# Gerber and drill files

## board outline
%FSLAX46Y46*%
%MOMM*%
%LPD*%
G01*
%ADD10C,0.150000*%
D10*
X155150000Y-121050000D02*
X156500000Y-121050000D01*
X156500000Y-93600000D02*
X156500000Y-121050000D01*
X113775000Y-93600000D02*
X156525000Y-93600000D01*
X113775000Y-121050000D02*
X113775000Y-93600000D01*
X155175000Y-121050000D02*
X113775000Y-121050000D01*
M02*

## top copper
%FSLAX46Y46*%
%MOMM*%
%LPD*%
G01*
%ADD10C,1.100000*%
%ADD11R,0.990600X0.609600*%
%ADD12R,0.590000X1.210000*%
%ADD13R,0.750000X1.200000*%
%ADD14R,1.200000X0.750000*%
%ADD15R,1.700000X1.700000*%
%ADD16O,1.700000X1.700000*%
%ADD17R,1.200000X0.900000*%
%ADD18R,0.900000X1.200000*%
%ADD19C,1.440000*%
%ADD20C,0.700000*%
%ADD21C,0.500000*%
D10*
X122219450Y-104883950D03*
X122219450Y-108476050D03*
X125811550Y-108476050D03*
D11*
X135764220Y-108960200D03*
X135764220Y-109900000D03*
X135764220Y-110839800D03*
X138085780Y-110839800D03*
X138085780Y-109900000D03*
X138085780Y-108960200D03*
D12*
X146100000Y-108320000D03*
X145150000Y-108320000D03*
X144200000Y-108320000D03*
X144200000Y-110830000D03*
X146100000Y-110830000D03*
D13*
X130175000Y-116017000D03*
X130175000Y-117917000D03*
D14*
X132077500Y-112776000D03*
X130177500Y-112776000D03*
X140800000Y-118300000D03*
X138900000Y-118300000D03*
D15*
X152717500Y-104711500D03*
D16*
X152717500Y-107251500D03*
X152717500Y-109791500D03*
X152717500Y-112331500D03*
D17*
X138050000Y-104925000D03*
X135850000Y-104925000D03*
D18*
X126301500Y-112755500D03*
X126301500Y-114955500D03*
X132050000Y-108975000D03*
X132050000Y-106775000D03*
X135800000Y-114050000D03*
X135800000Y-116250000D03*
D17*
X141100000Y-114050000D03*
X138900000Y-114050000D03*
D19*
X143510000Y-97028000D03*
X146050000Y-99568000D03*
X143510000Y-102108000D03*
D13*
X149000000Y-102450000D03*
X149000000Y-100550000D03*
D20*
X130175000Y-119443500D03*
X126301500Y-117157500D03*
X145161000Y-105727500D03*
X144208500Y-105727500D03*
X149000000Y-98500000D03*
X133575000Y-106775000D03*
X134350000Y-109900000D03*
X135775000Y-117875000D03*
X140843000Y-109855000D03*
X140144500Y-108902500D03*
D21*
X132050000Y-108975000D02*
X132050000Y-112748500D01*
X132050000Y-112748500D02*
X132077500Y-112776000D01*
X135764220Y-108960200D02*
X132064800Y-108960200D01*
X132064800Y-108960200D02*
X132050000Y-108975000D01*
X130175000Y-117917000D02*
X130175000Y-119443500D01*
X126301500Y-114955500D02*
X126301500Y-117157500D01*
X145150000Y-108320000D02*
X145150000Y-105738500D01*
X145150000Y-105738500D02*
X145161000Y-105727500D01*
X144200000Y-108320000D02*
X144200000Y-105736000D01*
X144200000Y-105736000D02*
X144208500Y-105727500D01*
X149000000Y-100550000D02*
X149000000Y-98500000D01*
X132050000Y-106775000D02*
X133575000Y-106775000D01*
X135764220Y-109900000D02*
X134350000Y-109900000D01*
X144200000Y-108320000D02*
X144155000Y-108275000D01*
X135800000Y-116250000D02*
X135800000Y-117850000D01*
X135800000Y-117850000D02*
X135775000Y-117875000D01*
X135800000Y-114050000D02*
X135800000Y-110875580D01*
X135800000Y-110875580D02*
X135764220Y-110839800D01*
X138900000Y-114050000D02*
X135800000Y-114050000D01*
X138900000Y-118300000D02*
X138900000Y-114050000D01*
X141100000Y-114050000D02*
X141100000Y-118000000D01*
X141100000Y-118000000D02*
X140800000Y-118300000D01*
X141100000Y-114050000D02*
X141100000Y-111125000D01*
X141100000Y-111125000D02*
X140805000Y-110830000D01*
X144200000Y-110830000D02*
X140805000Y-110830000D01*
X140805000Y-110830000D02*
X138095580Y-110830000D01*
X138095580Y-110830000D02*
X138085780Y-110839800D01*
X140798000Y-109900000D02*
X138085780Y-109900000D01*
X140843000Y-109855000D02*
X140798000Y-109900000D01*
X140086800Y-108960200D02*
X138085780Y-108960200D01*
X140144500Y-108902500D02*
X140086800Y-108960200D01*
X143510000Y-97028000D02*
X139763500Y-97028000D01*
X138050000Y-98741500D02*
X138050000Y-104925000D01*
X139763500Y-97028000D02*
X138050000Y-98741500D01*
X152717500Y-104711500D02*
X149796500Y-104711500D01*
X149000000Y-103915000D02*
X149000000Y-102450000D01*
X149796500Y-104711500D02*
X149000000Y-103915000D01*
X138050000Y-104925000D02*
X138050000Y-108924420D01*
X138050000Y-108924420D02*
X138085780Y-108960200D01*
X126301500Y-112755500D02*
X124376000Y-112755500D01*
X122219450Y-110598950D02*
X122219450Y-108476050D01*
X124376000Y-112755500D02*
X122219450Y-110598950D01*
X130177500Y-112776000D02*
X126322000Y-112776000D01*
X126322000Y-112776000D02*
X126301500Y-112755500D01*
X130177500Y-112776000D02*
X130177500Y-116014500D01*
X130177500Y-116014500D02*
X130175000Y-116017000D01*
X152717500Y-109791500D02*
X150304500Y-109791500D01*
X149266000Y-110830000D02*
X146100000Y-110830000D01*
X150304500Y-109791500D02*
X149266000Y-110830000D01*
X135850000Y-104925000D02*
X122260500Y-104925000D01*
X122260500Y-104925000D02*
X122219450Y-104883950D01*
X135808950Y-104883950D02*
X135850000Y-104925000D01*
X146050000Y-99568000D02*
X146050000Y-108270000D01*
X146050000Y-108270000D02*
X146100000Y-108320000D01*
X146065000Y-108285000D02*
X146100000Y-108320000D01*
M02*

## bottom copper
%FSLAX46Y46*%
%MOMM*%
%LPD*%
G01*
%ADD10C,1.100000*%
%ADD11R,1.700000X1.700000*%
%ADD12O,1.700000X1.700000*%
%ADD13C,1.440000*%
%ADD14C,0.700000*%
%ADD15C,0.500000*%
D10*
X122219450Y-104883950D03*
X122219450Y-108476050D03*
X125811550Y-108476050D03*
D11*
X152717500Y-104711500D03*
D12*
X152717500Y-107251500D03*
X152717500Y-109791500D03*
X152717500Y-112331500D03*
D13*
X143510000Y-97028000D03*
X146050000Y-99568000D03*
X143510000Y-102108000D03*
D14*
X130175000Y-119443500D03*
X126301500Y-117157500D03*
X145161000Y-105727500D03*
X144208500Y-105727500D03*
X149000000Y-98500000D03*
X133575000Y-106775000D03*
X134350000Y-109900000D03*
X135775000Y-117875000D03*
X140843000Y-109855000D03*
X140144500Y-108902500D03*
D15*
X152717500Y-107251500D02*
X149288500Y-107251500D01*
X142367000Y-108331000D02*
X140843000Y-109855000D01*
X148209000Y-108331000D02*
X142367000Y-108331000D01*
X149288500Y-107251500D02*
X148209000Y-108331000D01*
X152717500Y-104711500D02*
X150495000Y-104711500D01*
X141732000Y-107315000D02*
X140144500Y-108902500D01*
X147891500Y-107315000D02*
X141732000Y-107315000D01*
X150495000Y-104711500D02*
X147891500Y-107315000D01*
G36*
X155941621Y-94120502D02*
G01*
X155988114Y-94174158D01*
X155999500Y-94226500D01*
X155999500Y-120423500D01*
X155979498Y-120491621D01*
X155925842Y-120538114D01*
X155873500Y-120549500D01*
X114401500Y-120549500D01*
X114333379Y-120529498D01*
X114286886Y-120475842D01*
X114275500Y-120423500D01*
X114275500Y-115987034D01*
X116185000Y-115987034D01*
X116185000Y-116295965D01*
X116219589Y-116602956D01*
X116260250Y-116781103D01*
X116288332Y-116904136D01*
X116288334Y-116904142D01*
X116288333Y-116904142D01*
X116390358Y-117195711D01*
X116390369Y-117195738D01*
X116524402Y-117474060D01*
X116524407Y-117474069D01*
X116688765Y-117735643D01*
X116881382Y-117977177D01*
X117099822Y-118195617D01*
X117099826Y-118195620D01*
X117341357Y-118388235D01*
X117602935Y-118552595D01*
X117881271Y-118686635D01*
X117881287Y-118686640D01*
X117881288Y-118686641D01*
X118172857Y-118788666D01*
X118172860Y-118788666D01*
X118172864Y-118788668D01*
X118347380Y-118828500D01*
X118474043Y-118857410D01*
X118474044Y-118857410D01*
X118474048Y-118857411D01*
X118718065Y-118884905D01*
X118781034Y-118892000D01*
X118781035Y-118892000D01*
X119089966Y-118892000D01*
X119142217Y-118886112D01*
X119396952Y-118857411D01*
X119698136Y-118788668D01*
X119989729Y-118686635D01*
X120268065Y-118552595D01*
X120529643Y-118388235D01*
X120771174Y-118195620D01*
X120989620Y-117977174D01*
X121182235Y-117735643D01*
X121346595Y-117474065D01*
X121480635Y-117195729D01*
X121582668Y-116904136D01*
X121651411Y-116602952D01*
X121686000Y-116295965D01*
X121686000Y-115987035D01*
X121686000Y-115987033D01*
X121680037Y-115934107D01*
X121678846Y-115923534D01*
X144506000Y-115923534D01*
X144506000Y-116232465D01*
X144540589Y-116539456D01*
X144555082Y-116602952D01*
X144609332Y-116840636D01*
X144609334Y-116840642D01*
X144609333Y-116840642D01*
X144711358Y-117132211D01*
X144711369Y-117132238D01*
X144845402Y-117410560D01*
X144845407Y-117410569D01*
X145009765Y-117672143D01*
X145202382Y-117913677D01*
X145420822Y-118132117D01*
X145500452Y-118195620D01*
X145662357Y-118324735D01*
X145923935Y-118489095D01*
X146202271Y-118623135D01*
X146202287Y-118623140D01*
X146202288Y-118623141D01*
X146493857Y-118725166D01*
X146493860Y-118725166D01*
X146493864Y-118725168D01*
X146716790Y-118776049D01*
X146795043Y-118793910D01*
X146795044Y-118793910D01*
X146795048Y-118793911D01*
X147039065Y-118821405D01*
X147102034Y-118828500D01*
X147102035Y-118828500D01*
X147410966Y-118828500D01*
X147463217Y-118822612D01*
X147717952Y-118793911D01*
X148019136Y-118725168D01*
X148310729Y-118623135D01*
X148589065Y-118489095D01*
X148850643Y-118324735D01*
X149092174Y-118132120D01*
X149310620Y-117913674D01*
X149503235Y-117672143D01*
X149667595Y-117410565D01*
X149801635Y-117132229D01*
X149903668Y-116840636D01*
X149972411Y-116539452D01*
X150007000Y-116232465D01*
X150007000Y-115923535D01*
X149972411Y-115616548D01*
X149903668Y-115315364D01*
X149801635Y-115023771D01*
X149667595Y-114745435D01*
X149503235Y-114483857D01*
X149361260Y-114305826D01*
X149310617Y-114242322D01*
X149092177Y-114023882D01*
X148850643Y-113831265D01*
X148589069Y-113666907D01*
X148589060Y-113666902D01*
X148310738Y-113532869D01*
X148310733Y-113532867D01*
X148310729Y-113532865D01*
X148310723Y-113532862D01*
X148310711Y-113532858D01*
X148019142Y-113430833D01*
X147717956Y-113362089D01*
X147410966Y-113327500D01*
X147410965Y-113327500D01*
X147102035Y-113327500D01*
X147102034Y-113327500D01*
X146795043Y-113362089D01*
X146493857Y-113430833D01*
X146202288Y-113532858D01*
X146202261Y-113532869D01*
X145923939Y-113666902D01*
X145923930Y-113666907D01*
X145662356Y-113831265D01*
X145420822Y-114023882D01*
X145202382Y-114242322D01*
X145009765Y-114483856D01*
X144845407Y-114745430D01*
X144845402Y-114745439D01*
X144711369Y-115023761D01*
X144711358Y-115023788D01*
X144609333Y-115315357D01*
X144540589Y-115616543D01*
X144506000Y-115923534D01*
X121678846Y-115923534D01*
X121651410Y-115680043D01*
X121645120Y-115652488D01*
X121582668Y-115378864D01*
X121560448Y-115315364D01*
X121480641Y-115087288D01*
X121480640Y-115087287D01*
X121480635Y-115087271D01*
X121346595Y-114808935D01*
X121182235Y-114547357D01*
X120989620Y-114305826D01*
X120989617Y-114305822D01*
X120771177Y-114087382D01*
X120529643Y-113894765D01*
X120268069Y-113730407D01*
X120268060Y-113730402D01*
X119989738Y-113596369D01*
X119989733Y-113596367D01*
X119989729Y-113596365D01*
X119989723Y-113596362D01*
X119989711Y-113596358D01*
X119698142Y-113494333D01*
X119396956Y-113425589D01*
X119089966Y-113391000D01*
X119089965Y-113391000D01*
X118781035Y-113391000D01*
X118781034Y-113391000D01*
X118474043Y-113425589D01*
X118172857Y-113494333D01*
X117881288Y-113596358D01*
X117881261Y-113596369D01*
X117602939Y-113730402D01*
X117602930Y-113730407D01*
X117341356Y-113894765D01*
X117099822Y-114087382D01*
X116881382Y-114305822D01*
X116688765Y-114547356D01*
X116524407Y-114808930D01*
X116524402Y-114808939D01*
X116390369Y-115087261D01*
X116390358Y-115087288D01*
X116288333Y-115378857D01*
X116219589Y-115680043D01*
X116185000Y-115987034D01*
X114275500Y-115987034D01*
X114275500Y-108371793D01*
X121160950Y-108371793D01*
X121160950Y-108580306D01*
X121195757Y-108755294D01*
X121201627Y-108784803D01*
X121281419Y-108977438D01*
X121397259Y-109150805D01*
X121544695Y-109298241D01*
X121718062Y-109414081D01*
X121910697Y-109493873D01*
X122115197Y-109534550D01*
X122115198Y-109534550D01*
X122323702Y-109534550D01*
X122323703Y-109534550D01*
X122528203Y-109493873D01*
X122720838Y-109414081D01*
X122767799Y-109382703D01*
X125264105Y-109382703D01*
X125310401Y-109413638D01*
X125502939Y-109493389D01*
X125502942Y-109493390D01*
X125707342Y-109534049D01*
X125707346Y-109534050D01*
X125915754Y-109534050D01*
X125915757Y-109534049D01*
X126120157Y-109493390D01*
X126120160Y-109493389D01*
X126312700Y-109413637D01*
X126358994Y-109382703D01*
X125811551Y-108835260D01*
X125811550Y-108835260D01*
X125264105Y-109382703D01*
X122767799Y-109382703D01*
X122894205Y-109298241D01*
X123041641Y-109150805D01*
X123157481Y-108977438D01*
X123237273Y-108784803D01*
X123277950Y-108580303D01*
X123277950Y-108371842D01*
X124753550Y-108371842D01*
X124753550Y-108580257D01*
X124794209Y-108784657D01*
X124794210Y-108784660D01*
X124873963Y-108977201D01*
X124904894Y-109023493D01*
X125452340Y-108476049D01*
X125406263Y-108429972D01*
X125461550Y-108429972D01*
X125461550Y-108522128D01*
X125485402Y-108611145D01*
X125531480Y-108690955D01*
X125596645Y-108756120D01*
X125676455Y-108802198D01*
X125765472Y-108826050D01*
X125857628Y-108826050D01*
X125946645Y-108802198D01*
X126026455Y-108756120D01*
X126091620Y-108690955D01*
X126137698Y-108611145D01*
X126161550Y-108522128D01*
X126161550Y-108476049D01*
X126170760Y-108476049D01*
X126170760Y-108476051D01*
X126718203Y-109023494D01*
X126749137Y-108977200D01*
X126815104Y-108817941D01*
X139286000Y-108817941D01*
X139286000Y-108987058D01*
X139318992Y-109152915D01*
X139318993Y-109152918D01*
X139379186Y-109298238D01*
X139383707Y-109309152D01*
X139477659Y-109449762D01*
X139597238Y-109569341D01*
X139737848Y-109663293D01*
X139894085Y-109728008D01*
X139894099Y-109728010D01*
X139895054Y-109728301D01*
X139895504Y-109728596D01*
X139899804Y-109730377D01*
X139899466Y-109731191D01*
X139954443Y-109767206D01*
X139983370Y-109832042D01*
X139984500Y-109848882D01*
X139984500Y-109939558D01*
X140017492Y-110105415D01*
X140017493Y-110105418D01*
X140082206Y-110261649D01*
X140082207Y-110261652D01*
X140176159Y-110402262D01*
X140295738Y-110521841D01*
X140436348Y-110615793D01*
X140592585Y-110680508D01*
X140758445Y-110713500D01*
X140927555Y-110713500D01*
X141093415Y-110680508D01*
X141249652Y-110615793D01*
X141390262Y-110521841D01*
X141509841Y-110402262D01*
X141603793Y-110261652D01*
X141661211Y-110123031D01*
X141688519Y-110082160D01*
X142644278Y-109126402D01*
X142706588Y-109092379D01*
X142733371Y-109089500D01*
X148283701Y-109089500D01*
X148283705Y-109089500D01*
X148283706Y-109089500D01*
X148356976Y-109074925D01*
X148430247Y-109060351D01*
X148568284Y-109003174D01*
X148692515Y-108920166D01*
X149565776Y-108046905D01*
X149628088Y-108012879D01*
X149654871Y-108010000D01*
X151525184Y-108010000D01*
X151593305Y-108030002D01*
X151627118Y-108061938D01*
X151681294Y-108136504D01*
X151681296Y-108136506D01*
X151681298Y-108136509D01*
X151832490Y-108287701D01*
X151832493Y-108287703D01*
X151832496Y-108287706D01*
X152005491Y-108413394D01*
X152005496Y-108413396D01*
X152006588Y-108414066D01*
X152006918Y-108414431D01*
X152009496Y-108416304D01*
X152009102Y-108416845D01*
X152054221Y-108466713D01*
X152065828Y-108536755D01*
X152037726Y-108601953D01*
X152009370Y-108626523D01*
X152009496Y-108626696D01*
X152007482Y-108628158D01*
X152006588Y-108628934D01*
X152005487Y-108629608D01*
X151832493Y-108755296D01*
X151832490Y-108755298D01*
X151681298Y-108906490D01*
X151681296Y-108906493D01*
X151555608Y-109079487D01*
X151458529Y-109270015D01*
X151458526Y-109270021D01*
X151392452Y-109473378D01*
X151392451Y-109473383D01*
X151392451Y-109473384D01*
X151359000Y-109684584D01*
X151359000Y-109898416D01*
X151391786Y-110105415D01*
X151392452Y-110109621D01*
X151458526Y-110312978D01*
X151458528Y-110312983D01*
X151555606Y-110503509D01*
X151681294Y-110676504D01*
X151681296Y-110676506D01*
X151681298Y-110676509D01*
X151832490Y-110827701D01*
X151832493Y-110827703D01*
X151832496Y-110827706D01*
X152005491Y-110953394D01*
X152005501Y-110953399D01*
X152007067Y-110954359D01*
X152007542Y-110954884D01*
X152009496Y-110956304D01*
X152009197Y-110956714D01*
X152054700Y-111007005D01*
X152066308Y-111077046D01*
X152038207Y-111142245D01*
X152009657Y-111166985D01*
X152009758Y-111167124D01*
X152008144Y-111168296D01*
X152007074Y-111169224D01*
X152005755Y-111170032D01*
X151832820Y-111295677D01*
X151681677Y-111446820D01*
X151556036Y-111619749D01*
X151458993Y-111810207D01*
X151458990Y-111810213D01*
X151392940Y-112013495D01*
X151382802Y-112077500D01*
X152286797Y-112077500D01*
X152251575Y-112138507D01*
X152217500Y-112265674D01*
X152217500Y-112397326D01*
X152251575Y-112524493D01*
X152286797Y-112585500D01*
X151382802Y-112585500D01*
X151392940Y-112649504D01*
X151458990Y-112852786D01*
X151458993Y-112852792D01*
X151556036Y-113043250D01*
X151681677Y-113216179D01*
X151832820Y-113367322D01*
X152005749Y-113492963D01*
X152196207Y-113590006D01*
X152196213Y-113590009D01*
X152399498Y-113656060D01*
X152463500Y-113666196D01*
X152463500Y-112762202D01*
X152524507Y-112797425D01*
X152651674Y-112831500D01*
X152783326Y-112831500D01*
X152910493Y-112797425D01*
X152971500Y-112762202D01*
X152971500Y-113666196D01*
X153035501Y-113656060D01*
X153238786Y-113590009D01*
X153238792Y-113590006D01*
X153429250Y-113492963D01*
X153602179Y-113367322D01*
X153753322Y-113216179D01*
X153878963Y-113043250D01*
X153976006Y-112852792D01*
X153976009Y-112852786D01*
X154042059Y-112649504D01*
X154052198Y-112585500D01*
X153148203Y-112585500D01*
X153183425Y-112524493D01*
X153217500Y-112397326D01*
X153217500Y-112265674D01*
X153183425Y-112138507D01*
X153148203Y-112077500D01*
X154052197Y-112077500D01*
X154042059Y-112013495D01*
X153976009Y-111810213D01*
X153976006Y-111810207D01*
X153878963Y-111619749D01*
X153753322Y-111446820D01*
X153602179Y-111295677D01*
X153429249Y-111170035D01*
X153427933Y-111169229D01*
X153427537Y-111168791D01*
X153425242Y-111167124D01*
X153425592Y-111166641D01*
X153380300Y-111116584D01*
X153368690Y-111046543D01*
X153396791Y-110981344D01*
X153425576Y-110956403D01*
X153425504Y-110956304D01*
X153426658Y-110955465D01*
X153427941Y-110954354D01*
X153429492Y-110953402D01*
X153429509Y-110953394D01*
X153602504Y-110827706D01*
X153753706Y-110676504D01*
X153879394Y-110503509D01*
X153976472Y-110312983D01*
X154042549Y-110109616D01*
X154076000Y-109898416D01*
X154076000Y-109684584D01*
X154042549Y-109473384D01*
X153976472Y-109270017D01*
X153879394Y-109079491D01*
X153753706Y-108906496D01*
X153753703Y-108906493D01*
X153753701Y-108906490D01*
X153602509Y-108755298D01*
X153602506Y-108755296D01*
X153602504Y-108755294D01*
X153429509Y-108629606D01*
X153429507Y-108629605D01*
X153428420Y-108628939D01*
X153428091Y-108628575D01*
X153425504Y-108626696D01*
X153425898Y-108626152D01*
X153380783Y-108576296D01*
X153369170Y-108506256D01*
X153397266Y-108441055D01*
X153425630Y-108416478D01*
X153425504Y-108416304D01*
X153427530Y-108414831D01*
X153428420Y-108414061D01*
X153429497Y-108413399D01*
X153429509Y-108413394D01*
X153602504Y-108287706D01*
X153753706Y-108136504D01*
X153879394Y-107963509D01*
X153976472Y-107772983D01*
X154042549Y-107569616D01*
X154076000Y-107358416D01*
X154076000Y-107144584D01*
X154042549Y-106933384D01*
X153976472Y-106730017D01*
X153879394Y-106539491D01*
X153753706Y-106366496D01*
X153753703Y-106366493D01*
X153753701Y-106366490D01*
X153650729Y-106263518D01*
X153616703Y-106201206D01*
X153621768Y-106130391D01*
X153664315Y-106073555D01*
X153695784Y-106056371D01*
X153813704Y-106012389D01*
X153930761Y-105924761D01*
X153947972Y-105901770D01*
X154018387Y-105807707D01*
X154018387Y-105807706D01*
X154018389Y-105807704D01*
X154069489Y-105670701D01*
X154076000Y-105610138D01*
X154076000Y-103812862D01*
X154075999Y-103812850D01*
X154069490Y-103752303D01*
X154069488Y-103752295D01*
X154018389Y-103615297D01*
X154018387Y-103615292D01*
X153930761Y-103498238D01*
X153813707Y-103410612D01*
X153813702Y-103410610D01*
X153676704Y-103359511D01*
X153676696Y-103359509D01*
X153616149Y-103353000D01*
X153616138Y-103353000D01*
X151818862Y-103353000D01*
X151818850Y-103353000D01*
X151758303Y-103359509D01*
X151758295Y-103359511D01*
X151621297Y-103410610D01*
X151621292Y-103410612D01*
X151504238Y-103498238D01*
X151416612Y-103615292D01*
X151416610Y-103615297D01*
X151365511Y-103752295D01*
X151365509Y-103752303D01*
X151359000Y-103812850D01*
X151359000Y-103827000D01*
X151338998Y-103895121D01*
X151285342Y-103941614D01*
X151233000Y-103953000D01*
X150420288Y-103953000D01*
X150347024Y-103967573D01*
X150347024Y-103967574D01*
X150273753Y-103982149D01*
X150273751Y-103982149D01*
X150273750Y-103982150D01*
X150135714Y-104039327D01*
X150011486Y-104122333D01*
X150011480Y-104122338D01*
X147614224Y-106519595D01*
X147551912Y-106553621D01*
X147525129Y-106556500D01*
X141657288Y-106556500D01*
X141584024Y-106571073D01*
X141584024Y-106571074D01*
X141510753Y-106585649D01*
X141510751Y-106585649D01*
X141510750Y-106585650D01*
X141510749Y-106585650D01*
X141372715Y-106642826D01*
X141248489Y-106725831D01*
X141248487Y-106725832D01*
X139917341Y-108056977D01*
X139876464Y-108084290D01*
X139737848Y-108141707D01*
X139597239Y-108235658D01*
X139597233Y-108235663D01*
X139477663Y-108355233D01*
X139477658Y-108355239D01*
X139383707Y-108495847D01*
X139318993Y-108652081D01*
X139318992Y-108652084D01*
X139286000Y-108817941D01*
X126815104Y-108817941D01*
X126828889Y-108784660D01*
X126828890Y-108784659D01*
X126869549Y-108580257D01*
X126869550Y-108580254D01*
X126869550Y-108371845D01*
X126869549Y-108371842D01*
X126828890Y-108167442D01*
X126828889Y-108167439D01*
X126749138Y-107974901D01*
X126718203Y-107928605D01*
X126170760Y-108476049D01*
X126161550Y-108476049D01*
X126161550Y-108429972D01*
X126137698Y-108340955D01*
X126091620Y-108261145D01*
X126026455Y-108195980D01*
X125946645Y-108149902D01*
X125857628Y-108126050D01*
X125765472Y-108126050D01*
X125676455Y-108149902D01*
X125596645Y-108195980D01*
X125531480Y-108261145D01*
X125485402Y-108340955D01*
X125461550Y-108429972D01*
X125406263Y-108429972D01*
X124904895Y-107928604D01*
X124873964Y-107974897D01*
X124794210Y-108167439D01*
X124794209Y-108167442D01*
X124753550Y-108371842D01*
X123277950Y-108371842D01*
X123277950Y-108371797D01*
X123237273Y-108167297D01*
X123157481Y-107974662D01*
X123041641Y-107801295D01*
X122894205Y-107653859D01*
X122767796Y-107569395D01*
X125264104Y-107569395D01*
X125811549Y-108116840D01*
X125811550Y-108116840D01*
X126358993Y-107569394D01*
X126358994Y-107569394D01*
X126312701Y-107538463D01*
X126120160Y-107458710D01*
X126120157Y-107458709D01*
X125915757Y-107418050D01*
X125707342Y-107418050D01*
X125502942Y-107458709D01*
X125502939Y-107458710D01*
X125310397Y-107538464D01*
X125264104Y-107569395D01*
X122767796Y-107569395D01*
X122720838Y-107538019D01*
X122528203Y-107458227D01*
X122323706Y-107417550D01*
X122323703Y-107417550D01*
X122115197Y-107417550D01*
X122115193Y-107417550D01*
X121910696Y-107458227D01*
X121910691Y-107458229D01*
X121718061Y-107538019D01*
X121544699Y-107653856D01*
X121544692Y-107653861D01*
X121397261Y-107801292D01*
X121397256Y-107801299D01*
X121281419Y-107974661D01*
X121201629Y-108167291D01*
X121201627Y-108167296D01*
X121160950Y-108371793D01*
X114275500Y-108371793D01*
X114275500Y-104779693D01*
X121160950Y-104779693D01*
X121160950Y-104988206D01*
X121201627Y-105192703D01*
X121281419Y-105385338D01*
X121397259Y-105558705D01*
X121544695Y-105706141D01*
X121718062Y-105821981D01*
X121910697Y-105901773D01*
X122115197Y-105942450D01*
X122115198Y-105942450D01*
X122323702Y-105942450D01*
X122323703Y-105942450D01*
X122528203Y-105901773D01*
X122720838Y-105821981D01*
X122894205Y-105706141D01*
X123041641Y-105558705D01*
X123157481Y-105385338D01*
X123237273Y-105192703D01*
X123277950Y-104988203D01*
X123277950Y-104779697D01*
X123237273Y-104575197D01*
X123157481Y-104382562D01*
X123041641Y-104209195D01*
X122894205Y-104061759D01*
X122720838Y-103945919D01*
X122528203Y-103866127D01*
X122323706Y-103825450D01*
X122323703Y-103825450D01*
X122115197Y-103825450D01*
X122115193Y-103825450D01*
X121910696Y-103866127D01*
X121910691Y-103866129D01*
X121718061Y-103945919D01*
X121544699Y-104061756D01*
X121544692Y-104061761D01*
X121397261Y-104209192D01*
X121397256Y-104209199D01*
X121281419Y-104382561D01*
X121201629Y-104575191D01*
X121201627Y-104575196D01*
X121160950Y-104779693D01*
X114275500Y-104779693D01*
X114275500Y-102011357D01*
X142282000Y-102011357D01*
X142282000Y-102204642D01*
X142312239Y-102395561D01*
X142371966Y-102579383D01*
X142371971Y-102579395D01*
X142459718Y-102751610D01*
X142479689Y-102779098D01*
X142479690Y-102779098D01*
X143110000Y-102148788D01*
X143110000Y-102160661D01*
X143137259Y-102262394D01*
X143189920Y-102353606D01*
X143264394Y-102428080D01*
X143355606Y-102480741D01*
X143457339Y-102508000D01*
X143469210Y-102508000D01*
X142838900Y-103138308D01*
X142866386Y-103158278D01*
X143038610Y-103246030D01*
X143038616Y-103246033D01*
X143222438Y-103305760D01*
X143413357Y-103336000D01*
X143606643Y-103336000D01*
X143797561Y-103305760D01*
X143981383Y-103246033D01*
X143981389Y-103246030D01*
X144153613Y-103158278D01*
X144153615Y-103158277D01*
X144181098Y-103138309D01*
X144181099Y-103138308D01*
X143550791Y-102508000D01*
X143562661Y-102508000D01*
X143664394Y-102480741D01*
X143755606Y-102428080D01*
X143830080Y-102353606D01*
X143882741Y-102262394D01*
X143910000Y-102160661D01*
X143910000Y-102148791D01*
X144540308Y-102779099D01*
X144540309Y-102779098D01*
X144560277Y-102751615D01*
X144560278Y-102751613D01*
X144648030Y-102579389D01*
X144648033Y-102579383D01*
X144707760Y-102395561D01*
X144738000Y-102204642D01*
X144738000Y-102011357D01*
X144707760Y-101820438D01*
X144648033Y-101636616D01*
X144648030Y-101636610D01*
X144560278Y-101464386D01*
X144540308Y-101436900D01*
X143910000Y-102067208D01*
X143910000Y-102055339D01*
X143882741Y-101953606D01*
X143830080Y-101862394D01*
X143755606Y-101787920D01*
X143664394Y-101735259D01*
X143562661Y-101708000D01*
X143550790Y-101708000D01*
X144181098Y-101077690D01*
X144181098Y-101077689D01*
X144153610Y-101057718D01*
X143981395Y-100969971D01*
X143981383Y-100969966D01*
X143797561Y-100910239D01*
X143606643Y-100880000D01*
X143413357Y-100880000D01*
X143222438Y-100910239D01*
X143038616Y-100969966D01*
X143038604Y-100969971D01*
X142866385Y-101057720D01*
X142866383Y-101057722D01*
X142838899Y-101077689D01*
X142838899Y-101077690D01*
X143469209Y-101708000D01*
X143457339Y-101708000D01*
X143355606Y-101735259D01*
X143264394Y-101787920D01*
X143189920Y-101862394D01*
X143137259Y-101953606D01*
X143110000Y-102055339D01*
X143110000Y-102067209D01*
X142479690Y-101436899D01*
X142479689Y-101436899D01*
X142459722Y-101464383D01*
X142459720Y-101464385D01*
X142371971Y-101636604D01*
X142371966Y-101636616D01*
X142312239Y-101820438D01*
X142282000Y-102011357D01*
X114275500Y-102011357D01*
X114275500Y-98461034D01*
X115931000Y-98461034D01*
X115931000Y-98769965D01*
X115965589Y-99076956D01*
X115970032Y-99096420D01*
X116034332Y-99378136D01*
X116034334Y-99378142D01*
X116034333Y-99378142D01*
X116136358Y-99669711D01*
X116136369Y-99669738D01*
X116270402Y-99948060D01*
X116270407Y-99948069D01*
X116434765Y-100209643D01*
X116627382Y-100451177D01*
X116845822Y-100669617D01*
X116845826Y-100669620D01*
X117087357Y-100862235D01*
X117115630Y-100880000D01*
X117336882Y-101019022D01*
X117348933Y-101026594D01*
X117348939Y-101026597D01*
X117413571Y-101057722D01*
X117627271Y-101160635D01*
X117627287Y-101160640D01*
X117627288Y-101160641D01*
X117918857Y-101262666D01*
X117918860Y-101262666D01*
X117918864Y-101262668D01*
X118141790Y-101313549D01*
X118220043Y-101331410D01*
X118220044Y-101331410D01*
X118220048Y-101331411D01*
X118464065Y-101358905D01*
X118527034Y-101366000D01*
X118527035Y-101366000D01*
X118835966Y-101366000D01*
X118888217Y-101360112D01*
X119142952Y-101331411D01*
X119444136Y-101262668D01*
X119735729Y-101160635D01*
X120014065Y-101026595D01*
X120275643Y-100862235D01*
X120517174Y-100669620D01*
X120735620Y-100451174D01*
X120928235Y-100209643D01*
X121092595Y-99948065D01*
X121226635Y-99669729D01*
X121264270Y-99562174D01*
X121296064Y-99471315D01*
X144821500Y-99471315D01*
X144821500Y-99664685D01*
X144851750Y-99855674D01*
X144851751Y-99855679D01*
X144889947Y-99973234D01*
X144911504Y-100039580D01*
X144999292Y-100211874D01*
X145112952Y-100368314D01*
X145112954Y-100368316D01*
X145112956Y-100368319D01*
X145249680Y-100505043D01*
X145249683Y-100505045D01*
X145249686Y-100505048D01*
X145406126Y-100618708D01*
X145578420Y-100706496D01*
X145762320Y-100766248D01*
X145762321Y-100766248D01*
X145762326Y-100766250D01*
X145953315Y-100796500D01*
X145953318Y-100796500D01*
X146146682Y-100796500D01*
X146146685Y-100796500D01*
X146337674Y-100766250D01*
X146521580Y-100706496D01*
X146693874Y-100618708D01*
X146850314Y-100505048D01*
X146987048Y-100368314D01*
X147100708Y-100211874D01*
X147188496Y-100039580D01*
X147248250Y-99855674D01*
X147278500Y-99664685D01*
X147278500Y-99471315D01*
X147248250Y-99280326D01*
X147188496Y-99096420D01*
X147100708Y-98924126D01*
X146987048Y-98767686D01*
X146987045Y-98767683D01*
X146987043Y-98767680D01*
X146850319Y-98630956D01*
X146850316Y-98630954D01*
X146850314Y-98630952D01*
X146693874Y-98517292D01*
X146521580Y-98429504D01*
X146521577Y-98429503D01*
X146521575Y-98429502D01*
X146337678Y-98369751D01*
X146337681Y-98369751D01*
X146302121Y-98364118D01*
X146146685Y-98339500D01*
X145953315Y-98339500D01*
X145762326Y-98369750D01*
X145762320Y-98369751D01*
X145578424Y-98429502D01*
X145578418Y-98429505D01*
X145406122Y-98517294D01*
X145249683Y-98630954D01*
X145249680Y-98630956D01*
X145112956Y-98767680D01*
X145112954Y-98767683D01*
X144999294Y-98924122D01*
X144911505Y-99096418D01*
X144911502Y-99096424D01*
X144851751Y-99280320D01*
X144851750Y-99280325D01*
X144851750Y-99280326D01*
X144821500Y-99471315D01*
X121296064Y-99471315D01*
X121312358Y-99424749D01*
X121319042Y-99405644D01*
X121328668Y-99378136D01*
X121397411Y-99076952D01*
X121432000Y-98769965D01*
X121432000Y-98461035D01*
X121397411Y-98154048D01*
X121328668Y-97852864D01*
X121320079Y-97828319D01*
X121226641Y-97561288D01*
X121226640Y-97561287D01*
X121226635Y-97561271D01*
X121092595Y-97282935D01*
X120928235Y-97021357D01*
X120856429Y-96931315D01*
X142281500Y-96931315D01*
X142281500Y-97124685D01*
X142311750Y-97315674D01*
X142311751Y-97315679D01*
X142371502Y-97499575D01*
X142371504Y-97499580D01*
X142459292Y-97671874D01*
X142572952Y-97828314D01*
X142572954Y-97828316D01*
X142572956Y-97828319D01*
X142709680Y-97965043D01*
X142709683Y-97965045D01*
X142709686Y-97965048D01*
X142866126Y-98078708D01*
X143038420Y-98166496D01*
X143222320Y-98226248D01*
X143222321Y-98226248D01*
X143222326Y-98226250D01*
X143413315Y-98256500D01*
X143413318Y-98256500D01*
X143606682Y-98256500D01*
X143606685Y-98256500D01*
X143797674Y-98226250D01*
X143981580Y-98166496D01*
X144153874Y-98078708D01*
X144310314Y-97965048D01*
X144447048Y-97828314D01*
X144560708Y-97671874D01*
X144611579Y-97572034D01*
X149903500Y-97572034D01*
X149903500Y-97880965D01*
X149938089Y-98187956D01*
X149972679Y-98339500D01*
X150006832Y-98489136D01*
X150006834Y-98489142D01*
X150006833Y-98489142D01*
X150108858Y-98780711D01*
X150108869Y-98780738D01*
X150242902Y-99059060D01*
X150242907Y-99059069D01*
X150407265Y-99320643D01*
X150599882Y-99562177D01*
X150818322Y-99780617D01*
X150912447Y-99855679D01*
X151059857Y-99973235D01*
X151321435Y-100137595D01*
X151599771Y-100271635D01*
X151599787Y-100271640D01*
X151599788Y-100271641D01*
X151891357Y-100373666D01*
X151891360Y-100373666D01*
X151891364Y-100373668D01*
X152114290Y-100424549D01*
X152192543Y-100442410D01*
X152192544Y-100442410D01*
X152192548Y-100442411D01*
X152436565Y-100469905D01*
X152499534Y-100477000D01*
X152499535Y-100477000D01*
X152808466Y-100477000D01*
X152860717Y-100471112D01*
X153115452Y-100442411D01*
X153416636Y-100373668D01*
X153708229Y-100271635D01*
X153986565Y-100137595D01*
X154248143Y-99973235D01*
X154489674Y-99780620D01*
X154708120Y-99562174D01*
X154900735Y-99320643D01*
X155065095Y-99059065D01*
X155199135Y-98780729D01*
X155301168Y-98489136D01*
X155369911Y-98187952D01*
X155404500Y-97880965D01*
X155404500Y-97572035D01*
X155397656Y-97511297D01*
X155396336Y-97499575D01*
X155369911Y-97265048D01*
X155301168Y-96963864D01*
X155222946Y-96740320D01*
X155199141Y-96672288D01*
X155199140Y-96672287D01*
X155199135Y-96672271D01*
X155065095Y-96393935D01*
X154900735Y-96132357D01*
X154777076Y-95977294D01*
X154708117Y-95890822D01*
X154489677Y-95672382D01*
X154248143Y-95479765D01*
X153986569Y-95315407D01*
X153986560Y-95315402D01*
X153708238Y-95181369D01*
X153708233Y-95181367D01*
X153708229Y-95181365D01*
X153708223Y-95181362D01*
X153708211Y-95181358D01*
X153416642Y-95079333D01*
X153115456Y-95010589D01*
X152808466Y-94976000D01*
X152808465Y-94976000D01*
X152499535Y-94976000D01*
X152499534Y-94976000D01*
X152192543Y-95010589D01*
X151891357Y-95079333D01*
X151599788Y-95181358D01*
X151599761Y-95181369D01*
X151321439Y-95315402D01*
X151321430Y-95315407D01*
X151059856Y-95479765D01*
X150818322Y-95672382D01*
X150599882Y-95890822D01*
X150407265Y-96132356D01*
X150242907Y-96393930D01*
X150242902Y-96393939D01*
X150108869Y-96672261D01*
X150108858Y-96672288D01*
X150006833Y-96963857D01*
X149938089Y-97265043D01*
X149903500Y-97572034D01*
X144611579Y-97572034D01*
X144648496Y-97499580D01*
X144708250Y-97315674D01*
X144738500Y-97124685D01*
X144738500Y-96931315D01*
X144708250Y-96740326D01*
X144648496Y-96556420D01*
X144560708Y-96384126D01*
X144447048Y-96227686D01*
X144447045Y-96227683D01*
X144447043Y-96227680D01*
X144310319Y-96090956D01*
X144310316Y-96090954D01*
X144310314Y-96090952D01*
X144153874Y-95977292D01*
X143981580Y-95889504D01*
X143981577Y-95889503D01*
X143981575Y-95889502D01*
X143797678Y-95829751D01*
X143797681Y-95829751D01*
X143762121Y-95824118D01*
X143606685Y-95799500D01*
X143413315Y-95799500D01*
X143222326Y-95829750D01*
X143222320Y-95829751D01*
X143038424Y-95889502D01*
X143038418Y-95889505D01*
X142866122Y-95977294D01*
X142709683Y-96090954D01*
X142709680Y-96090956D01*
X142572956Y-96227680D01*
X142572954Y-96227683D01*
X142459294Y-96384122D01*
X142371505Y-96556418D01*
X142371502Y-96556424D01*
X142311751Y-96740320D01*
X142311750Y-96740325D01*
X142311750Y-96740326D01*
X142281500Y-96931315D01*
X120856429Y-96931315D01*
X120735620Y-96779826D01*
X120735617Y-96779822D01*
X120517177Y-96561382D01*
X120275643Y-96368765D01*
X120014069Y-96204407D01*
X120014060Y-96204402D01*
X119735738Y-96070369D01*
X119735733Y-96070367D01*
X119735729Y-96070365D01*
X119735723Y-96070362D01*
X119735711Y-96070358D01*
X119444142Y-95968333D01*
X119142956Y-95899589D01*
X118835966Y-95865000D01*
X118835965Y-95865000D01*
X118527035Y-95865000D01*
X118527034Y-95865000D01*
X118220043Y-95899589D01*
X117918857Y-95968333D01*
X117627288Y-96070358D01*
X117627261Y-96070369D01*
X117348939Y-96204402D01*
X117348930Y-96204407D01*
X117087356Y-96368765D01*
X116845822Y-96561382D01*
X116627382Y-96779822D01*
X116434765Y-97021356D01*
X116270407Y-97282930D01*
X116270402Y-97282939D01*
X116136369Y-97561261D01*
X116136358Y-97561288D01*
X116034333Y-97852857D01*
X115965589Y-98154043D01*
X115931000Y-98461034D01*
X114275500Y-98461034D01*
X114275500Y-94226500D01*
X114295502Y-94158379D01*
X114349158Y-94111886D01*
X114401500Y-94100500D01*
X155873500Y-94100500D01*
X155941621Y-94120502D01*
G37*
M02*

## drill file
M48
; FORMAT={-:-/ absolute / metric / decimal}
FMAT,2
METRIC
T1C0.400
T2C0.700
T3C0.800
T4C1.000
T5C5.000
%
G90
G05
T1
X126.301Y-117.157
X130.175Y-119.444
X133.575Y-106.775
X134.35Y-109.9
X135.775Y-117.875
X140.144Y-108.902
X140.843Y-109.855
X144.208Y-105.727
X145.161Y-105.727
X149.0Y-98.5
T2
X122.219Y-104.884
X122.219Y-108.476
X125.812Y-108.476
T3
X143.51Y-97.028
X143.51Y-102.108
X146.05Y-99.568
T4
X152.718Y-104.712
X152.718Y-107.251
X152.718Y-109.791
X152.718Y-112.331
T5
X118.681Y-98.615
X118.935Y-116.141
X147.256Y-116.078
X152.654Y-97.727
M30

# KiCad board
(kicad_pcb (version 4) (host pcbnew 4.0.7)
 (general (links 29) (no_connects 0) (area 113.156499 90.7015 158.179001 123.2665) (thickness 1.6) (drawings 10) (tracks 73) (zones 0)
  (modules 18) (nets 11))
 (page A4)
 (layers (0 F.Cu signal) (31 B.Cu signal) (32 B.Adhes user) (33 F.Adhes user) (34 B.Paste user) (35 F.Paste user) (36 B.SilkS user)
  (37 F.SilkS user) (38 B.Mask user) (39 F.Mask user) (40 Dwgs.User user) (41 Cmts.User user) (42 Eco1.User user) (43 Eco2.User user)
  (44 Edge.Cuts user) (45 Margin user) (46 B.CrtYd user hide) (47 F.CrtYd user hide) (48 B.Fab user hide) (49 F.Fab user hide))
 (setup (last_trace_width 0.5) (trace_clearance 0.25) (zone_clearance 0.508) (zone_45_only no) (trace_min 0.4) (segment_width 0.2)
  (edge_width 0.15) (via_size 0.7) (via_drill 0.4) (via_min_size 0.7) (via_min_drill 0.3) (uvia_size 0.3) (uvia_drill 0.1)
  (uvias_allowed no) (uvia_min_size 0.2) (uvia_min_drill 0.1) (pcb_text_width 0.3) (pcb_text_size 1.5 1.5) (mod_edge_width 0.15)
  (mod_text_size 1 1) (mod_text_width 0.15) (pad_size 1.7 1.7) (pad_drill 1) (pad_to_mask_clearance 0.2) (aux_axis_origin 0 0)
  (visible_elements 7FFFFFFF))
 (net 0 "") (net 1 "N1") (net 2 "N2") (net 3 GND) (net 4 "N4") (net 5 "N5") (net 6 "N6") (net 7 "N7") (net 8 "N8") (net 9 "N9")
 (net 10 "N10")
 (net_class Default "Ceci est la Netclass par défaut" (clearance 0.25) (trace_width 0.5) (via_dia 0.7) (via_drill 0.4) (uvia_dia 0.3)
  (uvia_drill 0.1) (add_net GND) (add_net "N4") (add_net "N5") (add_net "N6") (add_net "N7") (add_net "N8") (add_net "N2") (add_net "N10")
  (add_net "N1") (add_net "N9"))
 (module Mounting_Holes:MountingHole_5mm (layer F.Cu) (at 147.2565 116.078)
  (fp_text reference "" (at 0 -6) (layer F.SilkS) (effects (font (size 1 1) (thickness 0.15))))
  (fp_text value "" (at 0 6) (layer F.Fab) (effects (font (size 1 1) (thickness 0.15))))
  (pad 1 np_thru_hole circle (at 0 0) (size 5 5) (drill 5) (layers *.Cu *.Mask)))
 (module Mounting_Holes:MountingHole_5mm (layer F.Cu) (at 152.654 97.7265)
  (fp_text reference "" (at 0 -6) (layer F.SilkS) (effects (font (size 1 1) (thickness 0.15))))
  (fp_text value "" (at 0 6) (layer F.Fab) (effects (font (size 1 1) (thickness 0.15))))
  (pad 1 np_thru_hole circle (at 0 0) (size 5 5) (drill 5) (layers *.Cu *.Mask)))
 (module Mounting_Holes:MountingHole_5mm (layer F.Cu) (at 118.9355 116.1415)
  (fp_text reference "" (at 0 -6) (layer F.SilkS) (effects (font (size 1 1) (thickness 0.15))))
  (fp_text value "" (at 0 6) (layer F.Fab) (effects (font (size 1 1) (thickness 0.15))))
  (pad 1 np_thru_hole circle (at 0 0) (size 5 5) (drill 5) (layers *.Cu *.Mask)))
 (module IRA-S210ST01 (layer F.Cu) (at 124.0155 106.68 270)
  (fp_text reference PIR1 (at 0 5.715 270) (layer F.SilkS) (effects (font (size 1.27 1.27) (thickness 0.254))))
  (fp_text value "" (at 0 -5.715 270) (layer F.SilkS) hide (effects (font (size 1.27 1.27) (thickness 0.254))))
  (pad 1 thru_hole circle (at -1.79605 1.79605) (size 1.1 1.1) (drill 0.7) (layers *.Cu *.Mask F.SilkS) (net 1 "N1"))
  (pad 2 thru_hole circle (at 1.79605 1.79605) (size 1.1 1.1) (drill 0.7) (layers *.Cu *.Mask F.SilkS) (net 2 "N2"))
  (pad 3 thru_hole circle (at 1.79605 -1.79605) (size 1.1 1.1) (drill 0.7) (layers *.Cu *.Mask F.SilkS) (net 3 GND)))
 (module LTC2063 (layer F.Cu) (at 136.925 109.9)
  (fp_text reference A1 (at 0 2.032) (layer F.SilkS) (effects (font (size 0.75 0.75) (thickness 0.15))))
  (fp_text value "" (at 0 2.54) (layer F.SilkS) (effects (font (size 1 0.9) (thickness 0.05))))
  (pad 1 smd rect (at -1.16078 -0.9398) (size 0.9906 0.6096) (layers F.Cu F.Paste F.Mask) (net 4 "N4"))
  (pad 2 smd rect (at -1.16078 0) (size 0.9906 0.6096) (layers F.Cu F.Paste F.Mask) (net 3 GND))
  (pad 3 smd rect (at -1.16078 0.9398) (size 0.9906 0.6096) (layers F.Cu F.Paste F.Mask) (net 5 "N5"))
  (pad 4 smd rect (at 1.16078 0.9398) (size 0.9906 0.6096) (layers F.Cu F.Paste F.Mask) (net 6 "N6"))
  (pad 5 smd rect (at 1.16078 0) (size 0.9906 0.6096) (layers F.Cu F.Paste F.Mask) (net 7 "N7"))
  (pad 6 smd rect (at 1.16078 -0.9398) (size 0.9906 0.6096) (layers F.Cu F.Paste F.Mask) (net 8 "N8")))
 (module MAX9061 (layer F.Cu) (at 145.15 109.575 270)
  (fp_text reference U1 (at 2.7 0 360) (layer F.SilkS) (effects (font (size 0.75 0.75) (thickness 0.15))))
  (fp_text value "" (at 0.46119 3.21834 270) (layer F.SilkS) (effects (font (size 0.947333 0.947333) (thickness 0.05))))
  (pad 1 smd rect (at -1.255 -0.95 90) (size 1.21 0.59) (layers F.Cu F.Paste F.Mask) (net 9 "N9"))
  (pad 2 smd rect (at -1.255 0 90) (size 1.21 0.59) (layers F.Cu F.Paste F.Mask) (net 3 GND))
  (pad 3 smd rect (at -1.255 0.95 90) (size 1.21 0.59) (layers F.Cu F.Paste F.Mask) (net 3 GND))
  (pad 4 smd rect (at 1.255 0.95 270) (size 1.21 0.59) (layers F.Cu F.Paste F.Mask) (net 6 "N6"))
  (pad 5 smd rect (at 1.255 -0.95 270) (size 1.21 0.59) (layers F.Cu F.Paste F.Mask) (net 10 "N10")))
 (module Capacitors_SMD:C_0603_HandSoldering (layer F.Cu) (at 130.175 116.967 270)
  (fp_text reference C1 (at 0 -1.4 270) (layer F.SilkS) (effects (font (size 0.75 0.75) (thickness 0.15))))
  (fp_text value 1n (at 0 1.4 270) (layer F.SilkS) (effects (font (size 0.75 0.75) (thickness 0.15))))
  (pad 1 smd rect (at -0.95 0 270) (size 1.2 0.75) (layers F.Cu F.Paste F.Mask) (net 2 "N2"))
  (pad 2 smd rect (at 0.95 0 270) (size 1.2 0.75) (layers F.Cu F.Paste F.Mask) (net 3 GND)))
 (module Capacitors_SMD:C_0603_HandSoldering (layer F.Cu) (at 131.1275 112.776 180)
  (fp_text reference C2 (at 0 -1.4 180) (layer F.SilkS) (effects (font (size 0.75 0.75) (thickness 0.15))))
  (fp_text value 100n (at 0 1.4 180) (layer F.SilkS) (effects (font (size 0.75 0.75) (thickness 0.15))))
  (pad 1 smd rect (at -0.95 0 180) (size 1.2 0.75) (layers F.Cu F.Paste F.Mask) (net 4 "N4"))
  (pad 2 smd rect (at 0.95 0 180) (size 1.2 0.75) (layers F.Cu F.Paste F.Mask) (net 2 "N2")))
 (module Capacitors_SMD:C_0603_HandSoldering (layer F.Cu) (at 139.85 118.3 180)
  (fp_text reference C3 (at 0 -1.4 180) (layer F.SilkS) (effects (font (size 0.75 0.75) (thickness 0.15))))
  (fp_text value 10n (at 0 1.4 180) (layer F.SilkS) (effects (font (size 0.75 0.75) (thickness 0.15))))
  (pad 1 smd rect (at -0.95 0 180) (size 1.2 0.75) (layers F.Cu F.Paste F.Mask) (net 6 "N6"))
  (pad 2 smd rect (at 0.95 0 180) (size 1.2 0.75) (layers F.Cu F.Paste F.Mask) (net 5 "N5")))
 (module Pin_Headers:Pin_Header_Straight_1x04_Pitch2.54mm (layer F.Cu) (at 152.7175 104.7115)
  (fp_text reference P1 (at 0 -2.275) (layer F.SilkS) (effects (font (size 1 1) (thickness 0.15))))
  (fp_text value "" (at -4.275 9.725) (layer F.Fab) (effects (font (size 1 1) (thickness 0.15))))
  (pad 1 thru_hole rect (at 0 0) (size 1.7 1.7) (drill 1) (layers *.Cu *.Mask) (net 8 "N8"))
  (pad 2 thru_hole oval (at 0 2.54) (size 1.7 1.7) (drill 1) (layers *.Cu *.Mask) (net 7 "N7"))
  (pad 3 thru_hole oval (at 0 5.08) (size 1.7 1.7) (drill 1) (layers *.Cu *.Mask) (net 10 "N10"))
  (pad 4 thru_hole oval (at 0 7.62) (size 1.7 1.7) (drill 1) (layers *.Cu *.Mask) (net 3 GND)))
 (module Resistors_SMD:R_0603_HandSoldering (layer F.Cu) (at 136.95 104.925 180)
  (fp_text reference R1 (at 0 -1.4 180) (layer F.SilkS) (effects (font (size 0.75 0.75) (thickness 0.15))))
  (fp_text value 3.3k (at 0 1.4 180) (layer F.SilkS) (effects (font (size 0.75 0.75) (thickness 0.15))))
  (pad 1 smd rect (at -1.1 0 180) (size 1.2 0.9) (layers F.Cu F.Paste F.Mask) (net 8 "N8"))
  (pad 2 smd rect (at 1.1 0 180) (size 1.2 0.9) (layers F.Cu F.Paste F.Mask) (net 1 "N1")))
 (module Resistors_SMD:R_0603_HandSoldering (layer F.Cu) (at 126.3015 113.8555 270)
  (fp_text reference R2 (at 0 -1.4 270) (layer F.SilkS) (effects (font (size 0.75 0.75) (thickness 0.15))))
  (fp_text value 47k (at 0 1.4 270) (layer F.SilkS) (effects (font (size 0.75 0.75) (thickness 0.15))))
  (pad 1 smd rect (at -1.1 0 270) (size 1.2 0.9) (layers F.Cu F.Paste F.Mask) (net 2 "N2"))
  (pad 2 smd rect (at 1.1 0 270) (size 1.2 0.9) (layers F.Cu F.Paste F.Mask) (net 3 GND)))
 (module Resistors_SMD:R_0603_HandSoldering (layer F.Cu) (at 132.05 107.875 90)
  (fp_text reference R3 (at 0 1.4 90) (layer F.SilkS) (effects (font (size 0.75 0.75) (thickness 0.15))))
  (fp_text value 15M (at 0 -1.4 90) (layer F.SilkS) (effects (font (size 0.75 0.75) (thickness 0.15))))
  (pad 1 smd rect (at -1.1 0 90) (size 1.2 0.9) (layers F.Cu F.Paste F.Mask) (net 4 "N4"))
  (pad 2 smd rect (at 1.1 0 90) (size 1.2 0.9) (layers F.Cu F.Paste F.Mask) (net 3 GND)))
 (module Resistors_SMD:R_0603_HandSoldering (layer F.Cu) (at 135.8 115.15 270)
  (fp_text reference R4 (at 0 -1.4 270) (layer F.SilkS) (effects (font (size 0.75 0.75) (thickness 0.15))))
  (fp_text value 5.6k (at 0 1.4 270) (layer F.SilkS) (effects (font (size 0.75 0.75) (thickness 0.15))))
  (pad 1 smd rect (at -1.1 0 270) (size 1.2 0.9) (layers F.Cu F.Paste F.Mask) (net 5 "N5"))
  (pad 2 smd rect (at 1.1 0 270) (size 1.2 0.9) (layers F.Cu F.Paste F.Mask) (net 3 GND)))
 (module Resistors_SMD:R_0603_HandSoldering (layer F.Cu) (at 140 114.05 180)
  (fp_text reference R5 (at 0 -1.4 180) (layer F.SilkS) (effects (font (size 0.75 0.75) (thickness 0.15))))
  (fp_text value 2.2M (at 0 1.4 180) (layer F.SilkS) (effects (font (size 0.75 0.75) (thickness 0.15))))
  (pad 1 smd rect (at -1.1 0 180) (size 1.2 0.9) (layers F.Cu F.Paste F.Mask) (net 6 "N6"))
  (pad 2 smd rect (at 1.1 0 180) (size 1.2 0.9) (layers F.Cu F.Paste F.Mask) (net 5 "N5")))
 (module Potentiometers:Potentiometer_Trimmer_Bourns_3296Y (layer F.Cu) (at 143.51 97.028 90)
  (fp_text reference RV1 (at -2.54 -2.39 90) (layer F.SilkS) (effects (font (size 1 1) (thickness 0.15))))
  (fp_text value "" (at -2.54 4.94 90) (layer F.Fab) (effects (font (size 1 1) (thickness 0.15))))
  (pad 1 thru_hole circle (at 0 0 90) (size 1.44 1.44) (drill 0.8) (layers *.Cu *.Mask) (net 8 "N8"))
  (pad 2 thru_hole circle (at -2.54 2.54 90) (size 1.44 1.44) (drill 0.8) (layers *.Cu *.Mask) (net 9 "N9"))
  (pad 3 thru_hole circle (at -5.08 0 90) (size 1.44 1.44) (drill 0.8) (layers *.Cu *.Mask) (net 3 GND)))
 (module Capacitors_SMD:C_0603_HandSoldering (layer F.Cu) (at 149 101.5 90)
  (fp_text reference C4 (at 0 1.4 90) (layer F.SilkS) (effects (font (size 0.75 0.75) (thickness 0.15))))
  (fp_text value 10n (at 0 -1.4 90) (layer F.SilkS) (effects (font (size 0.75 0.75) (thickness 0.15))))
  (pad 1 smd rect (at -0.95 0 90) (size 1.2 0.75) (layers F.Cu F.Paste F.Mask) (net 8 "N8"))
  (pad 2 smd rect (at 0.95 0 90) (size 1.2 0.75) (layers F.Cu F.Paste F.Mask) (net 3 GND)))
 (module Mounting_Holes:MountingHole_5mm (layer F.Cu) (at 118.6815 98.6155)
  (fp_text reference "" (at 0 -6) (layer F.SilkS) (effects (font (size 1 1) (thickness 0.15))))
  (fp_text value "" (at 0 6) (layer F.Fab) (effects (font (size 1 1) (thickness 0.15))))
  (pad 1 np_thru_hole circle (at 0 0) (size 5 5) (drill 5) (layers *.Cu *.Mask)))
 (gr_line (start 155.15 121.05) (end 156.5 121.05) (angle 90) (layer Edge.Cuts) (width 0.15))
 (gr_line (start 156.5 93.6) (end 156.5 121.05) (angle 90) (layer Edge.Cuts) (width 0.15))
 (gr_line (start 113.775 93.6) (end 156.525 93.6) (angle 90) (layer Edge.Cuts) (width 0.15))
 (gr_line (start 113.775 121.05) (end 113.775 93.6) (angle 90) (layer Edge.Cuts) (width 0.15))
 (gr_line (start 155.175 121.05) (end 113.775 121.05) (angle 90) (layer Edge.Cuts) (width 0.15))
 (segment (start 132.05 108.975) (end 132.05 112.7485) (width 0.5) (layer F.Cu) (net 4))
 (segment (start 132.05 112.7485) (end 132.0775 112.776) (width 0.5) (layer F.Cu) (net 4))
 (segment (start 135.76422 108.9602) (end 132.0648 108.9602) (width 0.5) (layer F.Cu) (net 4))
 (segment (start 132.0648 108.9602) (end 132.05 108.975) (width 0.5) (layer F.Cu) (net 4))
 (segment (start 130.175 117.917) (end 130.175 119.4435) (width 0.5) (layer F.Cu) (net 3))
 (via (at 130.175 119.4435) (size 0.7) (drill 0.4) (layers F.Cu B.Cu) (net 3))
 (segment (start 126.3015 114.9555) (end 126.3015 117.1575) (width 0.5) (layer F.Cu) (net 3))
 (via (at 126.3015 117.1575) (size 0.7) (drill 0.4) (layers F.Cu B.Cu) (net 3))
 (segment (start 145.15 108.32) (end 145.15 105.7385) (width 0.5) (layer F.Cu) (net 3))
 (via (at 145.161 105.7275) (size 0.7) (drill 0.4) (layers F.Cu B.Cu) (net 3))
 (segment (start 145.15 105.7385) (end 145.161 105.7275) (width 0.5) (layer F.Cu) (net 3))
 (segment (start 144.2 108.32) (end 144.2 105.736) (width 0.5) (layer F.Cu) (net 3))
 (via (at 144.2085 105.7275) (size 0.7) (drill 0.4) (layers F.Cu B.Cu) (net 3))
 (segment (start 144.2 105.736) (end 144.2085 105.7275) (width 0.5) (layer F.Cu) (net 3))
 (segment (start 149 100.55) (end 149 98.5) (width 0.5) (layer F.Cu) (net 3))
 (via (at 149 98.5) (size 0.7) (drill 0.4) (layers F.Cu B.Cu) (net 3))
 (segment (start 132.05 106.775) (end 133.575 106.775) (width 0.5) (layer F.Cu) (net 3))
 (via (at 133.575 106.775) (size 0.7) (drill 0.4) (layers F.Cu B.Cu) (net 3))
 (segment (start 135.76422 109.9) (end 134.35 109.9) (width 0.5) (layer F.Cu) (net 3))
 (via (at 134.35 109.9) (size 0.7) (drill 0.4) (layers F.Cu B.Cu) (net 3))
 (segment (start 144.2 108.32) (end 144.155 108.275) (width 0.5) (layer F.Cu) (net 3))
 (segment (start 135.8 116.25) (end 135.8 117.85) (width 0.5) (layer F.Cu) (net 3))
 (via (at 135.775 117.875) (size 0.7) (drill 0.4) (layers F.Cu B.Cu) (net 3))
 (segment (start 135.8 117.85) (end 135.775 117.875) (width 0.5) (layer F.Cu) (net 3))
 (segment (start 135.8 114.05) (end 135.8 110.87558) (width 0.5) (layer F.Cu) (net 5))
 (segment (start 135.8 110.87558) (end 135.76422 110.8398) (width 0.5) (layer F.Cu) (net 5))
 (segment (start 138.9 114.05) (end 135.8 114.05) (width 0.5) (layer F.Cu) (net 5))
 (segment (start 138.9 118.3) (end 138.9 114.05) (width 0.5) (layer F.Cu) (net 5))
 (segment (start 141.1 114.05) (end 141.1 118) (width 0.5) (layer F.Cu) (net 6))
 (segment (start 141.1 118) (end 140.8 118.3) (width 0.5) (layer F.Cu) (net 6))
 (segment (start 141.1 114.05) (end 141.1 111.125) (width 0.5) (layer F.Cu) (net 6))
 (segment (start 141.1 111.125) (end 140.805 110.83) (width 0.5) (layer F.Cu) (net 6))
 (segment (start 144.2 110.83) (end 140.805 110.83) (width 0.5) (layer F.Cu) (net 6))
 (segment (start 140.805 110.83) (end 138.09558 110.83) (width 0.5) (layer F.Cu) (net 6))
 (segment (start 138.09558 110.83) (end 138.08578 110.8398) (width 0.5) (layer F.Cu) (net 6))
 (segment (start 152.7175 107.2515) (end 149.2885 107.2515) (width 0.5) (layer B.Cu) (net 7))
 (segment (start 140.798 109.9) (end 138.08578 109.9) (width 0.5) (layer F.Cu) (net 7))
 (segment (start 140.843 109.855) (end 140.798 109.9) (width 0.5) (layer F.Cu) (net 7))
 (via (at 140.843 109.855) (size 0.7) (drill 0.4) (layers F.Cu B.Cu) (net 7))
 (segment (start 142.367 108.331) (end 140.843 109.855) (width 0.5) (layer B.Cu) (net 7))
 (segment (start 148.209 108.331) (end 142.367 108.331) (width 0.5) (layer B.Cu) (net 7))
 (segment (start 149.2885 107.2515) (end 148.209 108.331) (width 0.5) (layer B.Cu) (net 7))
 (segment (start 152.7175 104.7115) (end 150.495 104.7115) (width 0.5) (layer B.Cu) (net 8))
 (segment (start 140.0868 108.9602) (end 138.08578 108.9602) (width 0.5) (layer F.Cu) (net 8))
 (segment (start 140.1445 108.9025) (end 140.0868 108.9602) (width 0.5) (layer F.Cu) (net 8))
 (via (at 140.1445 108.9025) (size 0.7) (drill 0.4) (layers F.Cu B.Cu) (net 8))
 (segment (start 141.732 107.315) (end 140.1445 108.9025) (width 0.5) (layer B.Cu) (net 8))
 (segment (start 147.8915 107.315) (end 141.732 107.315) (width 0.5) (layer B.Cu) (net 8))
 (segment (start 150.495 104.7115) (end 147.8915 107.315) (width 0.5) (layer B.Cu) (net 8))
 (segment (start 143.51 97.028) (end 139.7635 97.028) (width 0.5) (layer F.Cu) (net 8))
 (segment (start 138.05 98.7415) (end 138.05 104.925) (width 0.5) (layer F.Cu) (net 8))
 (segment (start 139.7635 97.028) (end 138.05 98.7415) (width 0.5) (layer F.Cu) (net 8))
 (segment (start 152.7175 104.7115) (end 149.7965 104.7115) (width 0.5) (layer F.Cu) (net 8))
 (segment (start 149 103.915) (end 149 102.45) (width 0.5) (layer F.Cu) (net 8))
 (segment (start 149.7965 104.7115) (end 149 103.915) (width 0.5) (layer F.Cu) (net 8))
 (segment (start 138.05 104.925) (end 138.05 108.92442) (width 0.5) (layer F.Cu) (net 8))
 (segment (start 138.05 108.92442) (end 138.08578 108.9602) (width 0.5) (layer F.Cu) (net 8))
 (segment (start 126.3015 112.7555) (end 124.376 112.7555) (width 0.5) (layer F.Cu) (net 2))
 (segment (start 122.21945 110.59895) (end 122.21945 108.47605) (width 0.5) (layer F.Cu) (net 2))
 (segment (start 124.376 112.7555) (end 122.21945 110.59895) (width 0.5) (layer F.Cu) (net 2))
 (segment (start 130.1775 112.776) (end 126.322 112.776) (width 0.5) (layer F.Cu) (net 2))
 (segment (start 126.322 112.776) (end 126.3015 112.7555) (width 0.5) (layer F.Cu) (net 2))
 (segment (start 130.1775 112.776) (end 130.1775 116.0145) (width 0.5) (layer F.Cu) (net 2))
 (segment (start 130.1775 116.0145) (end 130.175 116.017) (width 0.5) (layer F.Cu) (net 2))
 (segment (start 152.7175 109.7915) (end 150.3045 109.7915) (width 0.5) (layer F.Cu) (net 10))
 (segment (start 149.266 110.83) (end 146.1 110.83) (width 0.5) (layer F.Cu) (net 10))
 (segment (start 150.3045 109.7915) (end 149.266 110.83) (width 0.5) (layer F.Cu) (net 10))
 (segment (start 135.85 104.925) (end 122.2605 104.925) (width 0.5) (layer F.Cu) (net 1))
 (segment (start 122.2605 104.925) (end 122.21945 104.88395) (width 0.5) (layer F.Cu) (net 1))
 (segment (start 135.80895 104.88395) (end 135.85 104.925) (width 0.5) (layer F.Cu) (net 1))
 (segment (start 146.05 99.568) (end 146.05 108.27) (width 0.5) (layer F.Cu) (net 9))
 (segment (start 146.05 108.27) (end 146.1 108.32) (width 0.5) (layer F.Cu) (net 9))
 (segment (start 146.065 108.285) (end 146.1 108.32) (width 0.5) (layer F.Cu) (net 9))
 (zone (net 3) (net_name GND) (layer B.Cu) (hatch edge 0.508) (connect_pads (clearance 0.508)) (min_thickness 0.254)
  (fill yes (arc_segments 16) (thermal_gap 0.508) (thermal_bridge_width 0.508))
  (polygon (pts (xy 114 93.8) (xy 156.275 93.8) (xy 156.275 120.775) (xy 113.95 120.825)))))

